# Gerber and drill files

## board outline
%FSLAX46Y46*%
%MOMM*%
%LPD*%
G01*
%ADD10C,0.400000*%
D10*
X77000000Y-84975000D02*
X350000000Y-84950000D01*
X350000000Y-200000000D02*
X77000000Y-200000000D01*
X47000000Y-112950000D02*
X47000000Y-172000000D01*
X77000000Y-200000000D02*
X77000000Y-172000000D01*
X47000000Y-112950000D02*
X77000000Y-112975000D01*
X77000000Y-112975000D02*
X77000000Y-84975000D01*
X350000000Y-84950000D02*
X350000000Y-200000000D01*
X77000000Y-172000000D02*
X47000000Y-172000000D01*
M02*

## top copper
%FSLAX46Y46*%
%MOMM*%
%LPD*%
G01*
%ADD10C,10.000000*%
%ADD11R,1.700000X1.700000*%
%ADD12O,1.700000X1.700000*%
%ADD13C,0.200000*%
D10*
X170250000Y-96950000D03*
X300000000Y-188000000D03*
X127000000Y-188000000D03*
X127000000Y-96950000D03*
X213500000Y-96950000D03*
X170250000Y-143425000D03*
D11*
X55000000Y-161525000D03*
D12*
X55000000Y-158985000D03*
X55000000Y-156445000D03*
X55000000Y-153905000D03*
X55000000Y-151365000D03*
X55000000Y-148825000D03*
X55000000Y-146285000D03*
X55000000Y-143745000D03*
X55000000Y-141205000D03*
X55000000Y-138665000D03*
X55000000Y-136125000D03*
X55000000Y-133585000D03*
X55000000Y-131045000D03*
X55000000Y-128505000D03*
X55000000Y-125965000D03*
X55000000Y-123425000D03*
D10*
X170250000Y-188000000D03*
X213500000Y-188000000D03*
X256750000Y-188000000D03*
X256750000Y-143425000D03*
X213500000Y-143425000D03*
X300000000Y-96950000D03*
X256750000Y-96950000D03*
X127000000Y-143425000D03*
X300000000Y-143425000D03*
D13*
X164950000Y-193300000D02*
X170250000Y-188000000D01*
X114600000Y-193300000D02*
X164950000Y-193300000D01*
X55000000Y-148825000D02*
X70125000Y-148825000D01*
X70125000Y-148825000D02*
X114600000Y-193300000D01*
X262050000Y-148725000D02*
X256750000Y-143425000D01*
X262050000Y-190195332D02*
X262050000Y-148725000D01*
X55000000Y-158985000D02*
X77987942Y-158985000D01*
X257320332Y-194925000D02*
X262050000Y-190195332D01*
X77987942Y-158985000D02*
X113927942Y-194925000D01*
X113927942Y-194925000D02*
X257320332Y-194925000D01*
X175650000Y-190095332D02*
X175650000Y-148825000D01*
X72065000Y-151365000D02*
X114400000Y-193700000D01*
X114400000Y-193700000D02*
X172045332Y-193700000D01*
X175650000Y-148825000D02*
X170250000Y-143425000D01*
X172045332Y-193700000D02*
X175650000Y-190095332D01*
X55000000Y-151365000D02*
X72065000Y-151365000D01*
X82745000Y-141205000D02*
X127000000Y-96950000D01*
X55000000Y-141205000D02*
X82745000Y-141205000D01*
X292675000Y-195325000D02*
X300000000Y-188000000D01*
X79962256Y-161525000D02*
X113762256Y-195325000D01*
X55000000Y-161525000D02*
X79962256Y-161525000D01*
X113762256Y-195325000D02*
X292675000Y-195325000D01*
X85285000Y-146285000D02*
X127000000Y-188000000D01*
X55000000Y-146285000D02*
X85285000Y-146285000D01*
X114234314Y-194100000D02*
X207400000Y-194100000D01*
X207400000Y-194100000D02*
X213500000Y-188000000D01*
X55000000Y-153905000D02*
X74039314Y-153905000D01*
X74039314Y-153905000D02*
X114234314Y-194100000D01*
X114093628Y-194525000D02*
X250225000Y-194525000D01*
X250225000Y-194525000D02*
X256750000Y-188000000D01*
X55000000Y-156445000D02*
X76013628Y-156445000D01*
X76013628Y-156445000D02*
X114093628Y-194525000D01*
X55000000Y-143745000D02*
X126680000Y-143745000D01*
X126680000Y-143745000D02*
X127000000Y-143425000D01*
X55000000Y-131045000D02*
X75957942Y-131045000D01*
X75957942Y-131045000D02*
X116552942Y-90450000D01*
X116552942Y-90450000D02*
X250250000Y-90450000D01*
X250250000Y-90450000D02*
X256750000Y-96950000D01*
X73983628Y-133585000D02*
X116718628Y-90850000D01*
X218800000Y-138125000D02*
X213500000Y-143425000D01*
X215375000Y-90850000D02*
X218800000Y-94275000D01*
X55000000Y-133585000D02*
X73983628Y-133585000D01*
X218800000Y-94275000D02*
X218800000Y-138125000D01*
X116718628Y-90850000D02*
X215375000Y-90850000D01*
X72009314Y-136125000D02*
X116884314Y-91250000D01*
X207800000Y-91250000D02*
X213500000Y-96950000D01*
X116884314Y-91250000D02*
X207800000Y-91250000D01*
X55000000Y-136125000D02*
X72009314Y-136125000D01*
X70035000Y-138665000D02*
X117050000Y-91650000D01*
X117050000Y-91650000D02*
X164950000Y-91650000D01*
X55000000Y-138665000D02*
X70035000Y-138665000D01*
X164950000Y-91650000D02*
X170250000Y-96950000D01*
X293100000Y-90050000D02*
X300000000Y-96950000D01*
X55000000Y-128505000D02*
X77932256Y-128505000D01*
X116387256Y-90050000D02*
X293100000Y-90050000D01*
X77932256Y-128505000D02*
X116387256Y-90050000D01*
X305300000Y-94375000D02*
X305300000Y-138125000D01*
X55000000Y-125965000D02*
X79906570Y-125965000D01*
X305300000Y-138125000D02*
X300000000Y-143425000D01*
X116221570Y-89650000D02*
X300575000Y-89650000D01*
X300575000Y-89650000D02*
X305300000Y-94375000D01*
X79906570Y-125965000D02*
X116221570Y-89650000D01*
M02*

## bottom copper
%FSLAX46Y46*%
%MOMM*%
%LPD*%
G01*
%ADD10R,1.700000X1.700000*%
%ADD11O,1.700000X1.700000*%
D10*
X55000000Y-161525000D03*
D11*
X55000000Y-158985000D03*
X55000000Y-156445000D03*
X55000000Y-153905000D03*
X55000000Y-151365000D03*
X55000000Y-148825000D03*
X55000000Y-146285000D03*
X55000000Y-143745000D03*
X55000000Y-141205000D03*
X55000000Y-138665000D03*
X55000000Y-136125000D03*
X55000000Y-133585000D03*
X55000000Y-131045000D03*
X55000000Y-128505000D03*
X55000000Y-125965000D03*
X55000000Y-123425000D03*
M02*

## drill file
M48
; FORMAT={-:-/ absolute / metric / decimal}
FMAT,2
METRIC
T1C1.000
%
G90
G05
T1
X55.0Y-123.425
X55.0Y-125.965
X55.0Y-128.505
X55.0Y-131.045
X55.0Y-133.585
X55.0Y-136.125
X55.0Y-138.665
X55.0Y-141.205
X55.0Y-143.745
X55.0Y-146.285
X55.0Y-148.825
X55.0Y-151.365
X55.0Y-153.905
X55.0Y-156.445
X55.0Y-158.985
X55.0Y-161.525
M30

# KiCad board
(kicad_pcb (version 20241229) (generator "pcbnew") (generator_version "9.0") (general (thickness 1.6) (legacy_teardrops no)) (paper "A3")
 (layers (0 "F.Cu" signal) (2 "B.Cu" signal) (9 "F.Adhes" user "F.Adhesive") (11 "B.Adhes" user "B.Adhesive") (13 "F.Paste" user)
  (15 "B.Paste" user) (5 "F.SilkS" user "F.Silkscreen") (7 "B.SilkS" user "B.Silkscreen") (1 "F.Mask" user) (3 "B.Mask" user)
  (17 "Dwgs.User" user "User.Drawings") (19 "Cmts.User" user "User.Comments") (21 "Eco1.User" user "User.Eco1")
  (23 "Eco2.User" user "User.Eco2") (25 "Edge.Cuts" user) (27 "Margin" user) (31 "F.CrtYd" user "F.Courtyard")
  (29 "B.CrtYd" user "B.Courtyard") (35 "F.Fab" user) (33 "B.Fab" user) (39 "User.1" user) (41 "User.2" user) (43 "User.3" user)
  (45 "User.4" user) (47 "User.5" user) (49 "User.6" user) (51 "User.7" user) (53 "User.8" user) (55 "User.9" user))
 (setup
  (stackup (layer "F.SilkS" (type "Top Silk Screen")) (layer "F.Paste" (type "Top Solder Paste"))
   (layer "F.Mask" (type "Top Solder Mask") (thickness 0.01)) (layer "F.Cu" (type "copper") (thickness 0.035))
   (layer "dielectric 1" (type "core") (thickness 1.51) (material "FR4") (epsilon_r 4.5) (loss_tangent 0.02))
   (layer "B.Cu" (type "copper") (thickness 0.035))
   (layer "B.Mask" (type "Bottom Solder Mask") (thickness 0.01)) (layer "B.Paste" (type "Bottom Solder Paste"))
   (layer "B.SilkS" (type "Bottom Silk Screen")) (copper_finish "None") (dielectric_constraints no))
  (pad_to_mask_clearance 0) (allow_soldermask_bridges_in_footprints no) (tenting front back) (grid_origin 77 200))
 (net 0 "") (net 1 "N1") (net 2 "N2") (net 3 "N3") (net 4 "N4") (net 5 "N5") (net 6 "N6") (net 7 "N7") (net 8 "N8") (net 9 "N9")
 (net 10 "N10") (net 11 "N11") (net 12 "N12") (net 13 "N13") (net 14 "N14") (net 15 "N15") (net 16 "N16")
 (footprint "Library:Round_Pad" (layer "F.Cu") (at 170.25 96.95 180)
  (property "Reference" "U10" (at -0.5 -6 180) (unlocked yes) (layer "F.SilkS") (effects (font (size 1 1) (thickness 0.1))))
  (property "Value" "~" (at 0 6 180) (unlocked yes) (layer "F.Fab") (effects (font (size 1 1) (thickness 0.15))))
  (pad "1" smd circle (at 0 0 180) (size 10 10) (layers "F.Cu" "F.Mask" "F.Paste") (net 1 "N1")))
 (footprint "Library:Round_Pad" (layer "F.Cu") (at 300 188 180)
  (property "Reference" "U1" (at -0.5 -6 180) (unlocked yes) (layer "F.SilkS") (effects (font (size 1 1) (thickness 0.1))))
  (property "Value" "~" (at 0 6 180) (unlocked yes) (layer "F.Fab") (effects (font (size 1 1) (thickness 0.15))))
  (pad "1" smd circle (at 0 0 180) (size 10 10) (layers "F.Cu" "F.Mask" "F.Paste") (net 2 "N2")))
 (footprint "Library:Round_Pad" (layer "F.Cu") (at 127 188 180)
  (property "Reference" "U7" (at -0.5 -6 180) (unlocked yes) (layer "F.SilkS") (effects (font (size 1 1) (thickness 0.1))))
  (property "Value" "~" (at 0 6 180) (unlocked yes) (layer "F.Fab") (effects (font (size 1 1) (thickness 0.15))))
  (pad "1" smd circle (at 0 0 180) (size 10 10) (layers "F.Cu" "F.Mask" "F.Paste") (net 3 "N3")))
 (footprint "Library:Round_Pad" (layer "F.Cu") (at 127 96.95 180)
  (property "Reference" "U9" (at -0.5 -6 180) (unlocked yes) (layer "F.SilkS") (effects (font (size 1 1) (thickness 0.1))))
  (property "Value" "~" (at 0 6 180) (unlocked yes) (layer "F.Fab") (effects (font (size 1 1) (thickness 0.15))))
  (pad "1" smd circle (at 0 0 180) (size 10 10) (layers "F.Cu" "F.Mask" "F.Paste") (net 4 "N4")))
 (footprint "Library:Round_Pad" (layer "F.Cu") (at 213.5 96.95 180)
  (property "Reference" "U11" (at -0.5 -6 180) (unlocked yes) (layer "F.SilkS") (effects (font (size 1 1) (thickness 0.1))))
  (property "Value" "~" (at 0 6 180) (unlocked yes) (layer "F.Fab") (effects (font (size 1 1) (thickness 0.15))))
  (pad "1" smd circle (at 0 0 180) (size 10 10) (layers "F.Cu" "F.Mask" "F.Paste") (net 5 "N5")))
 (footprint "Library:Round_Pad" (layer "F.Cu") (at 170.25 143.425 180)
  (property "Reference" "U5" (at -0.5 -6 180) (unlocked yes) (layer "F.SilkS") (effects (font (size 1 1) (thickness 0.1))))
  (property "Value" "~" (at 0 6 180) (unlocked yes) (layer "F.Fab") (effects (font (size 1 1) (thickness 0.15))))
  (pad "1" smd circle (at 0 0 180) (size 10 10) (layers "F.Cu" "F.Mask" "F.Paste") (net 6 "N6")))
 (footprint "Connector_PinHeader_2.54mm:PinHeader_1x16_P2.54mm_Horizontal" (layer "F.Cu") (at 55 161.525 180)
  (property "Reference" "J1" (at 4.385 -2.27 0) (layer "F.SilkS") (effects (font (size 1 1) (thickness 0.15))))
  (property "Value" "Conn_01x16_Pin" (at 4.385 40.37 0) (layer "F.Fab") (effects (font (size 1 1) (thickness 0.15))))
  (pad "1" thru_hole rect (at 0 0 180) (size 1.7 1.7) (drill 1) (layers "*.Cu" "*.Mask") (remove_unused_layers no) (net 2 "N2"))
  (pad "2" thru_hole oval (at 0 2.54 180) (size 1.7 1.7) (drill 1) (layers "*.Cu" "*.Mask") (remove_unused_layers no) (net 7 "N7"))
  (pad "3" thru_hole oval (at 0 5.08 180) (size 1.7 1.7) (drill 1) (layers "*.Cu" "*.Mask") (remove_unused_layers no) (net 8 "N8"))
  (pad "4" thru_hole oval (at 0 7.62 180) (size 1.7 1.7) (drill 1) (layers "*.Cu" "*.Mask") (remove_unused_layers no) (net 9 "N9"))
  (pad "5" thru_hole oval (at 0 10.16 180) (size 1.7 1.7) (drill 1) (layers "*.Cu" "*.Mask") (remove_unused_layers no) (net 6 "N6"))
  (pad "6" thru_hole oval (at 0 12.7 180) (size 1.7 1.7) (drill 1) (layers "*.Cu" "*.Mask") (remove_unused_layers no) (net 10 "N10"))
  (pad "7" thru_hole oval (at 0 15.24 180) (size 1.7 1.7) (drill 1) (layers "*.Cu" "*.Mask") (remove_unused_layers no) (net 3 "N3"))
  (pad "8" thru_hole oval (at 0 17.78 180) (size 1.7 1.7) (drill 1) (layers "*.Cu" "*.Mask") (remove_unused_layers no) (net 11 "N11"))
  (pad "9" thru_hole oval (at 0 20.32 180) (size 1.7 1.7) (drill 1) (layers "*.Cu" "*.Mask") (remove_unused_layers no) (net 4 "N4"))
  (pad "10" thru_hole oval (at 0 22.86 180) (size 1.7 1.7) (drill 1) (layers "*.Cu" "*.Mask") (remove_unused_layers no) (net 1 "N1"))
  (pad "11" thru_hole oval (at 0 25.4 180) (size 1.7 1.7) (drill 1) (layers "*.Cu" "*.Mask") (remove_unused_layers no) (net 5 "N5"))
  (pad "12" thru_hole oval (at 0 27.94 180) (size 1.7 1.7) (drill 1) (layers "*.Cu" "*.Mask") (remove_unused_layers no) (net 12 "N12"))
  (pad "13" thru_hole oval (at 0 30.48 180) (size 1.7 1.7) (drill 1) (layers "*.Cu" "*.Mask") (remove_unused_layers no) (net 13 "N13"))
  (pad "14" thru_hole oval (at 0 33.02 180) (size 1.7 1.7) (drill 1) (layers "*.Cu" "*.Mask") (remove_unused_layers no) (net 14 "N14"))
  (pad "15" thru_hole oval (at 0 35.56 180) (size 1.7 1.7) (drill 1) (layers "*.Cu" "*.Mask") (remove_unused_layers no) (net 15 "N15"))
  (pad "16" thru_hole oval (at 0 38.1 180) (size 1.7 1.7) (drill 1) (layers "*.Cu" "*.Mask") (remove_unused_layers no) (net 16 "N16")))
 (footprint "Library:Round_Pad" (layer "F.Cu") (at 170.25 188 180)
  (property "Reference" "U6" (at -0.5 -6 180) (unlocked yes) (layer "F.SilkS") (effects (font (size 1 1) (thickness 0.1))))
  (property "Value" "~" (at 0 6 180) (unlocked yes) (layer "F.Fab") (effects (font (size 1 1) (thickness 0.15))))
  (pad "1" smd circle (at 0 0 180) (size 10 10) (layers "F.Cu" "F.Mask" "F.Paste") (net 10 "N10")))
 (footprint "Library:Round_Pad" (layer "F.Cu") (at 213.5 188 180)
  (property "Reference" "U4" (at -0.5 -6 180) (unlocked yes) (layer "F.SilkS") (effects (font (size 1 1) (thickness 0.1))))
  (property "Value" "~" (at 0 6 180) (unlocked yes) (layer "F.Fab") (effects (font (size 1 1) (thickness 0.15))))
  (pad "1" smd circle (at 0 0 180) (size 10 10) (layers "F.Cu" "F.Mask" "F.Paste") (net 9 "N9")))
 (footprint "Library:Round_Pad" (layer "F.Cu") (at 256.75 188 180)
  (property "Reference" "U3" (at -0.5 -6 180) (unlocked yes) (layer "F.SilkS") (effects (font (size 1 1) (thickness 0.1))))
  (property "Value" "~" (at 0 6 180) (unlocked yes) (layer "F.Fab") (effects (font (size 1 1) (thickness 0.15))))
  (pad "1" smd circle (at 0 0 180) (size 10 10) (layers "F.Cu" "F.Mask" "F.Paste") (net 8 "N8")))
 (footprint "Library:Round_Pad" (layer "F.Cu") (at 256.75 143.425 180)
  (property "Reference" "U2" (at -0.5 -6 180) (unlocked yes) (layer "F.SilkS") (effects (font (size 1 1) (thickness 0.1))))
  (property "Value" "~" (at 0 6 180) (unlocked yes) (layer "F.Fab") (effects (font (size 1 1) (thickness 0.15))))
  (pad "1" smd circle (at 0 0 180) (size 10 10) (layers "F.Cu" "F.Mask" "F.Paste") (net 7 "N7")))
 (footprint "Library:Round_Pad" (layer "F.Cu") (at 213.5 143.425 180)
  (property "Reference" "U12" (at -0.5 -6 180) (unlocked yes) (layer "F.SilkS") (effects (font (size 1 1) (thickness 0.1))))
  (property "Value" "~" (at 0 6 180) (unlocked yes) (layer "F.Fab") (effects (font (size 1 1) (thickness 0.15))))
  (pad "1" smd circle (at 0 0 180) (size 10 10) (layers "F.Cu" "F.Mask" "F.Paste") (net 12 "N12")))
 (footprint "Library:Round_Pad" (layer "F.Cu") (at 300 96.95 180)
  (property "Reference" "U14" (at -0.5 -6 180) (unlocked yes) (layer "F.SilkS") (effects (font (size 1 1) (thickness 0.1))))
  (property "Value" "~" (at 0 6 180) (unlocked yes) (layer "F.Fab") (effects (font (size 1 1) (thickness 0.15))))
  (pad "1" smd circle (at 0 0 180) (size 10 10) (layers "F.Cu" "F.Mask" "F.Paste") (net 14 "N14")))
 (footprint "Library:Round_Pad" (layer "F.Cu") (at 256.75 96.95 180)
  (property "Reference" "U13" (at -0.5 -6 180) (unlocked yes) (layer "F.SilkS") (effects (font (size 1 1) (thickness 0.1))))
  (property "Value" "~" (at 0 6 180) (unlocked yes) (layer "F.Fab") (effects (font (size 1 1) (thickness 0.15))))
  (pad "1" smd circle (at 0 0 180) (size 10 10) (layers "F.Cu" "F.Mask" "F.Paste") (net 13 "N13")))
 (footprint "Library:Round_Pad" (layer "F.Cu") (at 127 143.425 180)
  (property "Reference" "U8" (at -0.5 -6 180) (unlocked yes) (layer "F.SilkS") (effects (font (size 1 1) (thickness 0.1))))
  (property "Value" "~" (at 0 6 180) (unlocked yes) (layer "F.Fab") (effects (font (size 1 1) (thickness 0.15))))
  (pad "1" smd circle (at 0 0 180) (size 10 10) (layers "F.Cu" "F.Mask" "F.Paste") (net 11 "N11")))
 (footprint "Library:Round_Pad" (layer "F.Cu") (at 300 143.425 180)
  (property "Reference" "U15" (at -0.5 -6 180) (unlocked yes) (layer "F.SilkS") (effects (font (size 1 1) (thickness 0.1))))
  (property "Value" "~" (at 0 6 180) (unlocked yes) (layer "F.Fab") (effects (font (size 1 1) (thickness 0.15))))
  (pad "1" smd circle (at 0 0 180) (size 10 10) (layers "F.Cu" "F.Mask" "F.Paste") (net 15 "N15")))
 (gr_line (start 77 84.975) (end 350 84.95) (stroke (width 0.4) (type solid)) (layer "Edge.Cuts"))
 (gr_line (start 350 200) (end 77 200) (stroke (width 0.4) (type solid)) (layer "Edge.Cuts"))
 (gr_line (start 47 112.95) (end 47 172) (stroke (width 0.4) (type solid)) (layer "Edge.Cuts"))
 (gr_line (start 77 200) (end 77 172) (stroke (width 0.4) (type solid)) (layer "Edge.Cuts"))
 (gr_line (start 47 112.95) (end 77 112.975) (stroke (width 0.4) (type solid)) (layer "Edge.Cuts"))
 (gr_line (start 77 112.975) (end 77 84.975) (stroke (width 0.4) (type solid)) (layer "Edge.Cuts"))
 (gr_line (start 350 84.95) (end 350 200) (stroke (width 0.4) (type solid)) (layer "Edge.Cuts"))
 (gr_line (start 77 172) (end 47 172) (stroke (width 0.4) (type solid)) (layer "Edge.Cuts"))
 (segment (start 164.95 193.3) (end 170.25 188) (width 0.2) (layer "F.Cu") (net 10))
 (segment (start 114.6 193.3) (end 164.95 193.3) (width 0.2) (layer "F.Cu") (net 10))
 (segment (start 55 148.825) (end 70.125 148.825) (width 0.2) (layer "F.Cu") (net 10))
 (segment (start 70.125 148.825) (end 114.6 193.3) (width 0.2) (layer "F.Cu") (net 10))
 (segment (start 262.05 148.725) (end 256.75 143.425) (width 0.2) (layer "F.Cu") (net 7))
 (segment (start 262.05 190.195332) (end 262.05 148.725) (width 0.2) (layer "F.Cu") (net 7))
 (segment (start 55 158.985) (end 77.987942 158.985) (width 0.2) (layer "F.Cu") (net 7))
 (segment (start 257.320332 194.925) (end 262.05 190.195332) (width 0.2) (layer "F.Cu") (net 7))
 (segment (start 77.987942 158.985) (end 113.927942 194.925) (width 0.2) (layer "F.Cu") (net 7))
 (segment (start 113.927942 194.925) (end 257.320332 194.925) (width 0.2) (layer "F.Cu") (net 7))
 (segment (start 175.65 190.095332) (end 175.65 148.825) (width 0.2) (layer "F.Cu") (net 6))
 (segment (start 72.065 151.365) (end 114.4 193.7) (width 0.2) (layer "F.Cu") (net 6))
 (segment (start 114.4 193.7) (end 172.045332 193.7) (width 0.2) (layer "F.Cu") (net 6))
 (segment (start 175.65 148.825) (end 170.25 143.425) (width 0.2) (layer "F.Cu") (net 6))
 (segment (start 172.045332 193.7) (end 175.65 190.095332) (width 0.2) (layer "F.Cu") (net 6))
 (segment (start 55 151.365) (end 72.065 151.365) (width 0.2) (layer "F.Cu") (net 6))
 (segment (start 82.745 141.205) (end 127 96.95) (width 0.2) (layer "F.Cu") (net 4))
 (segment (start 55 141.205) (end 82.745 141.205) (width 0.2) (layer "F.Cu") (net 4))
 (segment (start 292.675 195.325) (end 300 188) (width 0.2) (layer "F.Cu") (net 2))
 (segment (start 79.962256 161.525) (end 113.762256 195.325) (width 0.2) (layer "F.Cu") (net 2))
 (segment (start 55 161.525) (end 79.962256 161.525) (width 0.2) (layer "F.Cu") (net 2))
 (segment (start 113.762256 195.325) (end 292.675 195.325) (width 0.2) (layer "F.Cu") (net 2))
 (segment (start 85.285 146.285) (end 127 188) (width 0.2) (layer "F.Cu") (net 3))
 (segment (start 55 146.285) (end 85.285 146.285) (width 0.2) (layer "F.Cu") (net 3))
 (segment (start 114.234314 194.1) (end 207.4 194.1) (width 0.2) (layer "F.Cu") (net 9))
 (segment (start 207.4 194.1) (end 213.5 188) (width 0.2) (layer "F.Cu") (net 9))
 (segment (start 55 153.905) (end 74.039314 153.905) (width 0.2) (layer "F.Cu") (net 9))
 (segment (start 74.039314 153.905) (end 114.234314 194.1) (width 0.2) (layer "F.Cu") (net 9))
 (segment (start 114.093628 194.525) (end 250.225 194.525) (width 0.2) (layer "F.Cu") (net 8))
 (segment (start 250.225 194.525) (end 256.75 188) (width 0.2) (layer "F.Cu") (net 8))
 (segment (start 55 156.445) (end 76.013628 156.445) (width 0.2) (layer "F.Cu") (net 8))
 (segment (start 76.013628 156.445) (end 114.093628 194.525) (width 0.2) (layer "F.Cu") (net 8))
 (segment (start 55 143.745) (end 126.68 143.745) (width 0.2) (layer "F.Cu") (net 11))
 (segment (start 126.68 143.745) (end 127 143.425) (width 0.2) (layer "F.Cu") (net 11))
 (segment (start 55 131.045) (end 75.957942 131.045) (width 0.2) (layer "F.Cu") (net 13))
 (segment (start 75.957942 131.045) (end 116.552942 90.45) (width 0.2) (layer "F.Cu") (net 13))
 (segment (start 116.552942 90.45) (end 250.25 90.45) (width 0.2) (layer "F.Cu") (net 13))
 (segment (start 250.25 90.45) (end 256.75 96.95) (width 0.2) (layer "F.Cu") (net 13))
 (segment (start 73.983628 133.585) (end 116.718628 90.85) (width 0.2) (layer "F.Cu") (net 12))
 (segment (start 218.8 138.125) (end 213.5 143.425) (width 0.2) (layer "F.Cu") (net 12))
 (segment (start 215.375 90.85) (end 218.8 94.275) (width 0.2) (layer "F.Cu") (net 12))
 (segment (start 55 133.585) (end 73.983628 133.585) (width 0.2) (layer "F.Cu") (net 12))
 (segment (start 218.8 94.275) (end 218.8 138.125) (width 0.2) (layer "F.Cu") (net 12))
 (segment (start 116.718628 90.85) (end 215.375 90.85) (width 0.2) (layer "F.Cu") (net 12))
 (segment (start 72.009314 136.125) (end 116.884314 91.25) (width 0.2) (layer "F.Cu") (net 5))
 (segment (start 207.8 91.25) (end 213.5 96.95) (width 0.2) (layer "F.Cu") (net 5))
 (segment (start 116.884314 91.25) (end 207.8 91.25) (width 0.2) (layer "F.Cu") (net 5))
 (segment (start 55 136.125) (end 72.009314 136.125) (width 0.2) (layer "F.Cu") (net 5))
 (segment (start 70.035 138.665) (end 117.05 91.65) (width 0.2) (layer "F.Cu") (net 1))
 (segment (start 117.05 91.65) (end 164.95 91.65) (width 0.2) (layer "F.Cu") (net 1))
 (segment (start 55 138.665) (end 70.035 138.665) (width 0.2) (layer "F.Cu") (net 1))
 (segment (start 164.95 91.65) (end 170.25 96.95) (width 0.2) (layer "F.Cu") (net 1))
 (segment (start 293.1 90.05) (end 300 96.95) (width 0.2) (layer "F.Cu") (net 14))
 (segment (start 55 128.505) (end 77.932256 128.505) (width 0.2) (layer "F.Cu") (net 14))
 (segment (start 116.387256 90.05) (end 293.1 90.05) (width 0.2) (layer "F.Cu") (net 14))
 (segment (start 77.932256 128.505) (end 116.387256 90.05) (width 0.2) (layer "F.Cu") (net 14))
 (segment (start 305.3 94.375) (end 305.3 138.125) (width 0.2) (layer "F.Cu") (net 15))
 (segment (start 55 125.965) (end 79.90657 125.965) (width 0.2) (layer "F.Cu") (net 15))
 (segment (start 305.3 138.125) (end 300 143.425) (width 0.2) (layer "F.Cu") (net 15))
 (segment (start 116.22157 89.65) (end 300.575 89.65) (width 0.2) (layer "F.Cu") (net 15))
 (segment (start 300.575 89.65) (end 305.3 94.375) (width 0.2) (layer "F.Cu") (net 15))
 (segment (start 79.90657 125.965) (end 116.22157 89.65) (width 0.2) (layer "F.Cu") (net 15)))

